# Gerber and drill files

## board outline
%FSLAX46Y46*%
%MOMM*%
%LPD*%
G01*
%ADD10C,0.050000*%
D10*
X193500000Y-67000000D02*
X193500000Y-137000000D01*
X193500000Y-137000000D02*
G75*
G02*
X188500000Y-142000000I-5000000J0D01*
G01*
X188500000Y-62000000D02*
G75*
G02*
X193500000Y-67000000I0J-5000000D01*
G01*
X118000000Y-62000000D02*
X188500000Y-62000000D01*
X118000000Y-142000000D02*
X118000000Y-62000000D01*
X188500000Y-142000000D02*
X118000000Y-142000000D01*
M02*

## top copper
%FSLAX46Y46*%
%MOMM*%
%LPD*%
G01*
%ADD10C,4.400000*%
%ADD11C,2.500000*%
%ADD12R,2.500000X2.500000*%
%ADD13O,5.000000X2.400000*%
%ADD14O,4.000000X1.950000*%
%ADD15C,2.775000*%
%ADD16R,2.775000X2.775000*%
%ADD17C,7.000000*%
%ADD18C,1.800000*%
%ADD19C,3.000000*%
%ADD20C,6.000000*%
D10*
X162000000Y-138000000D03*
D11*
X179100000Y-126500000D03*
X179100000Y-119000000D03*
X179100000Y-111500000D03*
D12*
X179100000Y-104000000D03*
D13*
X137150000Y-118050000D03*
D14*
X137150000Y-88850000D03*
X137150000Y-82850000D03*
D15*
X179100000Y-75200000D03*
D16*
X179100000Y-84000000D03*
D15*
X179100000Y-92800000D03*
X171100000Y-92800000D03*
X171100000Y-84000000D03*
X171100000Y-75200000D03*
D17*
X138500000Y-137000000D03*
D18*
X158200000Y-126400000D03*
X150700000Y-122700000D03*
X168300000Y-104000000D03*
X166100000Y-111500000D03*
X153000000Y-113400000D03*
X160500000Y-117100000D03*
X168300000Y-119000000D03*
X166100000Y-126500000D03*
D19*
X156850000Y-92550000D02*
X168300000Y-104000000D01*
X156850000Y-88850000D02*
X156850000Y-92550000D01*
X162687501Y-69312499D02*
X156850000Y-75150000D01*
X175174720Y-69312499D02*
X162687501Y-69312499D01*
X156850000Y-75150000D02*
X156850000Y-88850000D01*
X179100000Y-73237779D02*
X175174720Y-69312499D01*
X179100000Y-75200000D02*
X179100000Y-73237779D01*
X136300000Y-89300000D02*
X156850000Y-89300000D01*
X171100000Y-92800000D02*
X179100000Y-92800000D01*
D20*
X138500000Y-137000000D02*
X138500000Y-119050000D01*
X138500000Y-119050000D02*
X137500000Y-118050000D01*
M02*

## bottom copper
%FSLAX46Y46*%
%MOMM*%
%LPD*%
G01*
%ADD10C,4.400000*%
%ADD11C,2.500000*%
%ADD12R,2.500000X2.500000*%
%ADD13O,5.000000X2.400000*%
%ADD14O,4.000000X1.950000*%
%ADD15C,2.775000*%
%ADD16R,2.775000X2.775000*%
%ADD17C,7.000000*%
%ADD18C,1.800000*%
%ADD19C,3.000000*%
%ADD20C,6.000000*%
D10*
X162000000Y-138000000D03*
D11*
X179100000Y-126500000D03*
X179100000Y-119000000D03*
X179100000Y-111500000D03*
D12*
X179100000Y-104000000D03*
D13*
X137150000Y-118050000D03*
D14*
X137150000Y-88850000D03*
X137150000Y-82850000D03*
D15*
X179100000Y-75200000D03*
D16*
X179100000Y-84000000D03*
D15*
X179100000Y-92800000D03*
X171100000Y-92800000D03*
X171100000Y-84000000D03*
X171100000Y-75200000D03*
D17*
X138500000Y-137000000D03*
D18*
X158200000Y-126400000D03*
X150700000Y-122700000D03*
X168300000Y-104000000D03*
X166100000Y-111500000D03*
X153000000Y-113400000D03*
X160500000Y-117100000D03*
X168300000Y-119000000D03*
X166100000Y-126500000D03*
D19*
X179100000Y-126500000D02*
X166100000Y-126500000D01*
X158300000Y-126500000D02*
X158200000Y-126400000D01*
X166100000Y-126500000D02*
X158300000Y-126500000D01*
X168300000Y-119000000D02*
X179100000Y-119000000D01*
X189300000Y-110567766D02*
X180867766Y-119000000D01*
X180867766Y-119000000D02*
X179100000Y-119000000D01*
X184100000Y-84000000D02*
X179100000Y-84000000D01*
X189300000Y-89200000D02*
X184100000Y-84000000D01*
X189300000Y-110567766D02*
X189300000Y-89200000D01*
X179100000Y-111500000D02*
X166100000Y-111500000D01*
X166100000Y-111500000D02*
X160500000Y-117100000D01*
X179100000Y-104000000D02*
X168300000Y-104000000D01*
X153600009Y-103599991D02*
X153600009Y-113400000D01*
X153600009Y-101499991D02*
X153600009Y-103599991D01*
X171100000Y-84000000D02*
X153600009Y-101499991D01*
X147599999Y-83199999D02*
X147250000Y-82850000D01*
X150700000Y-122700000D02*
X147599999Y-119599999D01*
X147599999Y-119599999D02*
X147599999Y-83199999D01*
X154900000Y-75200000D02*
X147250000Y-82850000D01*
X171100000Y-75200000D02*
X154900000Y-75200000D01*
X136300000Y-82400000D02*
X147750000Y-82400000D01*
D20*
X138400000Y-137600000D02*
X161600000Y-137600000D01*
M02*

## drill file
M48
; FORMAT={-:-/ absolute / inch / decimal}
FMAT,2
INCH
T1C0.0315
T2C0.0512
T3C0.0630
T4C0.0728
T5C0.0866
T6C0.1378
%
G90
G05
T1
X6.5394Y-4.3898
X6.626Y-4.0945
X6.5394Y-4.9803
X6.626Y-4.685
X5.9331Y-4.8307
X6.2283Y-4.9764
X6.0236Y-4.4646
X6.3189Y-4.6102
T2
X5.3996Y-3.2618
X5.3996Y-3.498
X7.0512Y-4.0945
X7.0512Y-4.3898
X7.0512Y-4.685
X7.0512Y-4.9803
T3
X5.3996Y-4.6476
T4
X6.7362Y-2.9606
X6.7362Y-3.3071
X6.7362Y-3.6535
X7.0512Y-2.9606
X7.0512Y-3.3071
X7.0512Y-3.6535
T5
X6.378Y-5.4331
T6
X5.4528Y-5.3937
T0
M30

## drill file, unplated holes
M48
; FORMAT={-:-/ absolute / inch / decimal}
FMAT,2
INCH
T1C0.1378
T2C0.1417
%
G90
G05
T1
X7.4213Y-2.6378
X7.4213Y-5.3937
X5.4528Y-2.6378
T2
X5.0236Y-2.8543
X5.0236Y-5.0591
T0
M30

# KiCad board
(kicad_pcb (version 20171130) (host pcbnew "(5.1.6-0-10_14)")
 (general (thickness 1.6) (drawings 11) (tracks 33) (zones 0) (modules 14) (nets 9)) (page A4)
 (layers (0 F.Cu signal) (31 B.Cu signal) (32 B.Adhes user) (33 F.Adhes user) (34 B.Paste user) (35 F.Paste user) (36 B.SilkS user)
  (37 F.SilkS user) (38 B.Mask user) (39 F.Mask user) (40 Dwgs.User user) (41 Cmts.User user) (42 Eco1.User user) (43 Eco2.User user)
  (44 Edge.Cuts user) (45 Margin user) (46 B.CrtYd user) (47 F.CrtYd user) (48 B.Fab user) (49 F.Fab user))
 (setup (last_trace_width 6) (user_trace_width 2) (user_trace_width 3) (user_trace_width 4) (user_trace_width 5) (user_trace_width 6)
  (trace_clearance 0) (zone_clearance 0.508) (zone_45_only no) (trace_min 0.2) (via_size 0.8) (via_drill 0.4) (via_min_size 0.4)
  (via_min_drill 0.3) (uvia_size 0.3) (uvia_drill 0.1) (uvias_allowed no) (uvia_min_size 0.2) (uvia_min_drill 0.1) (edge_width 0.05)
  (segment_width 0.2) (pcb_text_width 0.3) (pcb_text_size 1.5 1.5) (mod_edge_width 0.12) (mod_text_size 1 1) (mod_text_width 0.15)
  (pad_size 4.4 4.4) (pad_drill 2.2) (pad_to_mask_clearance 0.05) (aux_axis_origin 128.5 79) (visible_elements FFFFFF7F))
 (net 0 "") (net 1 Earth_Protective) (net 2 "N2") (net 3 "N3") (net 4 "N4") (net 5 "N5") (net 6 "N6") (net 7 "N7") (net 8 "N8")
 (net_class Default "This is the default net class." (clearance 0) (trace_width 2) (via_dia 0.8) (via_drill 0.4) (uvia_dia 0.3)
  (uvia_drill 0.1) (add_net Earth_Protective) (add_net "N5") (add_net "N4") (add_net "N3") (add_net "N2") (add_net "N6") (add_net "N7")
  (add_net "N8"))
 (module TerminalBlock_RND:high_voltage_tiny (layer F.Cu) (at 180.5 138.5)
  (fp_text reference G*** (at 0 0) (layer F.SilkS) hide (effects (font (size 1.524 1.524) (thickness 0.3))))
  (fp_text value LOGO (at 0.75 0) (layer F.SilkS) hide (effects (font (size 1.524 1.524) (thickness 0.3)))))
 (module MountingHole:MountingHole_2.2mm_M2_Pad (layer F.Cu) (at 162 138)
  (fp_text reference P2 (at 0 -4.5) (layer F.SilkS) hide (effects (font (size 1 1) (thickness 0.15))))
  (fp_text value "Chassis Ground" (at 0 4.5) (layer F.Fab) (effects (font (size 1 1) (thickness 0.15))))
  (pad 1 thru_hole circle (at 0 0) (size 4.4 4.4) (drill 2.2) (layers *.Cu *.Mask) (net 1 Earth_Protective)))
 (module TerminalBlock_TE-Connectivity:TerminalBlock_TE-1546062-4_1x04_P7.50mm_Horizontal (layer F.Cu) (at 179.1 104 270) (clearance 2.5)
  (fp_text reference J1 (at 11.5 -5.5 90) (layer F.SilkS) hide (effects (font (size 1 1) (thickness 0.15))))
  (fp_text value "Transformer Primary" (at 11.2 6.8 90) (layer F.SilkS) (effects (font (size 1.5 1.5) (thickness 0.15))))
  (pad 4 thru_hole circle (at 22.5 0 270) (size 2.5 2.5) (drill 1.3) (layers *.Cu *.Mask) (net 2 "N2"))
  (pad 3 thru_hole circle (at 15 0 270) (size 2.5 2.5) (drill 1.3) (layers *.Cu *.Mask) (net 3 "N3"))
  (pad 2 thru_hole circle (at 7.5 0 270) (size 2.5 2.5) (drill 1.3) (layers *.Cu *.Mask) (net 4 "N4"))
  (pad 1 thru_hole rect (at 0 0 270) (size 2.5 2.5) (drill 1.3) (layers *.Cu *.Mask) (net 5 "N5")))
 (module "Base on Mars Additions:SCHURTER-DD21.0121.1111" (layer F.Cu) (at 127.6 100.5 270)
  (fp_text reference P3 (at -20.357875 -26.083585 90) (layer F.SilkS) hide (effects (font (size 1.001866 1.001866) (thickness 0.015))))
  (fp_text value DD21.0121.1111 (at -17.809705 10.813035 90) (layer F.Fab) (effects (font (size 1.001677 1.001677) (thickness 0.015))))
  (pad PE thru_hole oval (at 17.55 -9.55 270) (size 2.4 5) (drill 1.6) (layers *.Cu *.Mask) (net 1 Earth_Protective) (clearance 6))
  (pad N thru_hole oval (at -11.65 -9.55 270) (size 1.95 4) (drill 1.3) (layers *.Cu *.Mask) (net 5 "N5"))
  (pad L thru_hole oval (at -17.65 -9.55 270) (size 1.95 4) (drill 1.3) (layers *.Cu *.Mask) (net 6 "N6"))
  (pad None np_thru_hole circle (at 28 0 270) (size 3.6 3.6) (drill 3.6) (layers *.Cu *.Mask))
  (pad None np_thru_hole circle (at -28 0 270) (size 3.6 3.6) (drill 3.6) (layers *.Cu *.Mask)))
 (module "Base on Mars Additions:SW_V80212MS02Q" (layer F.Cu) (at 175.1 84 180)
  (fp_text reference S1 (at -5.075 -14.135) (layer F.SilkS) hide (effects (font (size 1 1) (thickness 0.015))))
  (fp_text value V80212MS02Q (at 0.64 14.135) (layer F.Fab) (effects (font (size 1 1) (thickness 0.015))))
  (pad 1A thru_hole circle (at -4 8.8 180) (size 2.775 2.775) (drill 1.85) (layers *.Cu *.Mask) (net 5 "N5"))
  (pad 1 thru_hole rect (at -4 0 180) (size 2.775 2.775) (drill 1.85) (layers *.Cu *.Mask) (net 3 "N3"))
  (pad 1B thru_hole circle (at -4 -8.8 180) (size 2.775 2.775) (drill 1.85) (layers *.Cu *.Mask) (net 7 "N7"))
  (pad 2B thru_hole circle (at 4 -8.8 180) (size 2.775 2.775) (drill 1.85) (layers *.Cu *.Mask) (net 7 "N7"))
  (pad 2 thru_hole circle (at 4 0 180) (size 2.775 2.775) (drill 1.85) (layers *.Cu *.Mask) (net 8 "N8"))
  (pad 2A thru_hole circle (at 4 8.8 180) (size 2.775 2.775) (drill 1.85) (layers *.Cu *.Mask) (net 6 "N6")))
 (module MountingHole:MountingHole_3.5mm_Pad (layer F.Cu) (at 138.5 137)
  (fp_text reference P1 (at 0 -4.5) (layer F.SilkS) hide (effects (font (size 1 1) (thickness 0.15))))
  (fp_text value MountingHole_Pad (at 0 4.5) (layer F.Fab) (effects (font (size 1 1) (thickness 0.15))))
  (pad 1 thru_hole circle (at 0 0) (size 7 7) (drill 3.5) (layers *.Cu *.Mask) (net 1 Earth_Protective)))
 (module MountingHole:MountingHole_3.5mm (layer F.Cu) (at 188.5 67)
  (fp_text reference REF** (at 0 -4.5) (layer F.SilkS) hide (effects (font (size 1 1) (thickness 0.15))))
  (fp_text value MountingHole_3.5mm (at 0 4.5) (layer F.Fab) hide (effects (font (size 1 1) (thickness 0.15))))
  (pad 1 np_thru_hole circle (at 0 0) (size 3.5 3.5) (drill 3.5) (layers *.Cu *.Mask)))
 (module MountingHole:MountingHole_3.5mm (layer F.Cu) (at 188.5 137)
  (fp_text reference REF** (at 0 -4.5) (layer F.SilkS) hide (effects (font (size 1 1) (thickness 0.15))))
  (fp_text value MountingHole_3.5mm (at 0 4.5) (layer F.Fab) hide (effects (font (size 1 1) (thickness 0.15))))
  (pad 1 np_thru_hole circle (at 0 0) (size 3.5 3.5) (drill 3.5) (layers *.Cu *.Mask)))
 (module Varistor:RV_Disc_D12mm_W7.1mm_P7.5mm (layer F.Cu) (at 158.2 126.4 180)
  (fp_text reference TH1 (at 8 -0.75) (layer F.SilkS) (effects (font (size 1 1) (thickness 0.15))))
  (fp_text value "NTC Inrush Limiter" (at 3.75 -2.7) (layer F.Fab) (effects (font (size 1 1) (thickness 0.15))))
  (pad 1 thru_hole circle (at 0 0 180) (size 1.8 1.8) (drill 0.8) (layers *.Cu *.Mask) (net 2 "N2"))
  (pad 2 thru_hole circle (at 7.5 3.7 180) (size 1.8 1.8) (drill 0.8) (layers *.Cu *.Mask) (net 6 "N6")))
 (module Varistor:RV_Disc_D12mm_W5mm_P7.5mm (layer F.Cu) (at 166.1 111.5 90)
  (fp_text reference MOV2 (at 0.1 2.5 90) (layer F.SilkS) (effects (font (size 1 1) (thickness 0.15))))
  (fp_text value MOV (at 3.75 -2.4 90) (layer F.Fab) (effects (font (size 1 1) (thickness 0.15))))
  (pad 2 thru_hole circle (at 7.5 2.2 90) (size 1.8 1.8) (drill 0.8) (layers *.Cu *.Mask) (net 5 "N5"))
  (pad 1 thru_hole circle (at 0 0 90) (size 1.8 1.8) (drill 0.8) (layers *.Cu *.Mask) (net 4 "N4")))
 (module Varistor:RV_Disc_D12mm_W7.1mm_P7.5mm (layer F.Cu) (at 153 113.4)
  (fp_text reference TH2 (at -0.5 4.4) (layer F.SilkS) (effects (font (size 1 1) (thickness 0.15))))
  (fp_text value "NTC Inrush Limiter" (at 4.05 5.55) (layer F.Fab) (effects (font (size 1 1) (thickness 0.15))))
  (pad 1 thru_hole circle (at 0 0) (size 1.8 1.8) (drill 0.8) (layers *.Cu *.Mask) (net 8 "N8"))
  (pad 2 thru_hole circle (at 7.5 3.7) (size 1.8 1.8) (drill 0.8) (layers *.Cu *.Mask) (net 4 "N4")))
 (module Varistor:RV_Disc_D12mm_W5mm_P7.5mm (layer F.Cu) (at 166.1 126.5 90)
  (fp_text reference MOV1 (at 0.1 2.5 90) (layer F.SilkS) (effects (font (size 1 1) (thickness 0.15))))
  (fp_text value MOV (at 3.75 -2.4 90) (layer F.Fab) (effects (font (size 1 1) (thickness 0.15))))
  (pad 2 thru_hole circle (at 7.5 2.2 90) (size 1.8 1.8) (drill 0.8) (layers *.Cu *.Mask) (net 3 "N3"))
  (pad 1 thru_hole circle (at 0 0 90) (size 1.8 1.8) (drill 0.8) (layers *.Cu *.Mask) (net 2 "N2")))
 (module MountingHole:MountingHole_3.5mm (layer F.Cu) (at 138.5 67) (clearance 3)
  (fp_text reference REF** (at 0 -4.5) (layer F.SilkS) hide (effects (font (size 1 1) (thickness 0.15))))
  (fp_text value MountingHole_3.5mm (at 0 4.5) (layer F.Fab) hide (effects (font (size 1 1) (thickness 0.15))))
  (pad 1 np_thru_hole circle (at 0 0) (size 3.5 3.5) (drill 3.5) (layers *.Cu *.Mask)))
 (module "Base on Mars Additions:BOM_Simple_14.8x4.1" (layer F.Cu) (at 174.2 67.2)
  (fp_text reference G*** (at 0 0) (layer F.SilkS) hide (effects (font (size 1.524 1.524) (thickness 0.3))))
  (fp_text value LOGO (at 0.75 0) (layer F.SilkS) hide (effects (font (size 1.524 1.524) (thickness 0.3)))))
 (gr_line (start 193.5 67) (end 193.5 137) (layer Edge.Cuts) (width 0.05))
 (gr_arc (start 188.5 137) (end 188.5 142) (angle -90) (layer Edge.Cuts) (width 0.05))
 (gr_arc (start 188.5 67) (end 193.5 67) (angle -90) (layer Edge.Cuts) (width 0.05))
 (gr_line (start 118 62) (end 188.5 62) (layer Edge.Cuts) (width 0.05))
 (gr_line (start 118 142) (end 118 62) (layer Edge.Cuts) (width 0.05))
 (gr_line (start 188.5 142) (end 118 142) (layer Edge.Cuts) (width 0.05))
 (segment (start 179.1 126.5) (end 166.1 126.5) (width 3) (layer B.Cu) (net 2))
 (segment (start 158.3 126.5) (end 158.2 126.4) (width 3) (layer B.Cu) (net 2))
 (segment (start 166.1 126.5) (end 158.3 126.5) (width 3) (layer B.Cu) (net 2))
 (segment (start 168.3 119) (end 179.1 119) (width 3) (layer B.Cu) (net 3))
 (segment (start 189.3 110.567766) (end 180.867766 119) (width 3) (layer B.Cu) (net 3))
 (segment (start 180.867766 119) (end 179.1 119) (width 3) (layer B.Cu) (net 3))
 (segment (start 184.1 84) (end 179.1 84) (width 3) (layer B.Cu) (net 3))
 (segment (start 189.3 89.2) (end 184.1 84) (width 3) (layer B.Cu) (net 3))
 (segment (start 189.3 110.567766) (end 189.3 89.2) (width 3) (layer B.Cu) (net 3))
 (segment (start 179.1 111.5) (end 166.1 111.5) (width 3) (layer B.Cu) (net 4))
 (segment (start 166.1 111.5) (end 160.5 117.1) (width 3) (layer B.Cu) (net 4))
 (segment (start 156.85 92.55) (end 168.3 104) (width 3) (layer F.Cu) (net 5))
 (segment (start 156.85 88.85) (end 156.85 92.55) (width 3) (layer F.Cu) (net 5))
 (segment (start 179.1 104) (end 168.3 104) (width 3) (layer B.Cu) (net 5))
 (segment (start 162.687501 69.312499) (end 156.85 75.15) (width 3) (layer F.Cu) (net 5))
 (segment (start 175.17472 69.312499) (end 162.687501 69.312499) (width 3) (layer F.Cu) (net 5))
 (segment (start 156.85 75.15) (end 156.85 88.85) (width 3) (layer F.Cu) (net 5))
 (segment (start 179.1 73.237779) (end 175.17472 69.312499) (width 3) (layer F.Cu) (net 5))
 (segment (start 179.1 75.2) (end 179.1 73.237779) (width 3) (layer F.Cu) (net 5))
 (segment (start 136.3 89.3) (end 156.85 89.3) (width 3) (layer F.Cu) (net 5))
 (segment (start 171.1 92.8) (end 179.1 92.8) (width 3) (layer F.Cu) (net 7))
 (segment (start 153.600009 103.599991) (end 153.600009 113.4) (width 3) (layer B.Cu) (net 8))
 (segment (start 153.600009 101.499991) (end 153.600009 103.599991) (width 3) (layer B.Cu) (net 8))
 (segment (start 171.1 84) (end 153.600009 101.499991) (width 3) (layer B.Cu) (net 8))
 (segment (start 147.599999 83.199999) (end 147.25 82.85) (width 3) (layer B.Cu) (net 6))
 (segment (start 150.7 122.7) (end 147.599999 119.599999) (width 3) (layer B.Cu) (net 6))
 (segment (start 147.599999 119.599999) (end 147.599999 83.199999) (width 3) (layer B.Cu) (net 6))
 (segment (start 154.9 75.2) (end 147.25 82.85) (width 3) (layer B.Cu) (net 6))
 (segment (start 171.1 75.2) (end 154.9 75.2) (width 3) (layer B.Cu) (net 6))
 (segment (start 136.3 82.4) (end 147.75 82.4) (width 3) (layer B.Cu) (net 6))
 (segment (start 138.4 137.6) (end 161.6 137.6) (width 6) (layer B.Cu) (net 1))
 (segment (start 138.5 137) (end 138.5 119.05) (width 6) (layer F.Cu) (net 1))
 (segment (start 138.5 119.05) (end 137.5 118.05) (width 6) (layer F.Cu) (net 1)))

